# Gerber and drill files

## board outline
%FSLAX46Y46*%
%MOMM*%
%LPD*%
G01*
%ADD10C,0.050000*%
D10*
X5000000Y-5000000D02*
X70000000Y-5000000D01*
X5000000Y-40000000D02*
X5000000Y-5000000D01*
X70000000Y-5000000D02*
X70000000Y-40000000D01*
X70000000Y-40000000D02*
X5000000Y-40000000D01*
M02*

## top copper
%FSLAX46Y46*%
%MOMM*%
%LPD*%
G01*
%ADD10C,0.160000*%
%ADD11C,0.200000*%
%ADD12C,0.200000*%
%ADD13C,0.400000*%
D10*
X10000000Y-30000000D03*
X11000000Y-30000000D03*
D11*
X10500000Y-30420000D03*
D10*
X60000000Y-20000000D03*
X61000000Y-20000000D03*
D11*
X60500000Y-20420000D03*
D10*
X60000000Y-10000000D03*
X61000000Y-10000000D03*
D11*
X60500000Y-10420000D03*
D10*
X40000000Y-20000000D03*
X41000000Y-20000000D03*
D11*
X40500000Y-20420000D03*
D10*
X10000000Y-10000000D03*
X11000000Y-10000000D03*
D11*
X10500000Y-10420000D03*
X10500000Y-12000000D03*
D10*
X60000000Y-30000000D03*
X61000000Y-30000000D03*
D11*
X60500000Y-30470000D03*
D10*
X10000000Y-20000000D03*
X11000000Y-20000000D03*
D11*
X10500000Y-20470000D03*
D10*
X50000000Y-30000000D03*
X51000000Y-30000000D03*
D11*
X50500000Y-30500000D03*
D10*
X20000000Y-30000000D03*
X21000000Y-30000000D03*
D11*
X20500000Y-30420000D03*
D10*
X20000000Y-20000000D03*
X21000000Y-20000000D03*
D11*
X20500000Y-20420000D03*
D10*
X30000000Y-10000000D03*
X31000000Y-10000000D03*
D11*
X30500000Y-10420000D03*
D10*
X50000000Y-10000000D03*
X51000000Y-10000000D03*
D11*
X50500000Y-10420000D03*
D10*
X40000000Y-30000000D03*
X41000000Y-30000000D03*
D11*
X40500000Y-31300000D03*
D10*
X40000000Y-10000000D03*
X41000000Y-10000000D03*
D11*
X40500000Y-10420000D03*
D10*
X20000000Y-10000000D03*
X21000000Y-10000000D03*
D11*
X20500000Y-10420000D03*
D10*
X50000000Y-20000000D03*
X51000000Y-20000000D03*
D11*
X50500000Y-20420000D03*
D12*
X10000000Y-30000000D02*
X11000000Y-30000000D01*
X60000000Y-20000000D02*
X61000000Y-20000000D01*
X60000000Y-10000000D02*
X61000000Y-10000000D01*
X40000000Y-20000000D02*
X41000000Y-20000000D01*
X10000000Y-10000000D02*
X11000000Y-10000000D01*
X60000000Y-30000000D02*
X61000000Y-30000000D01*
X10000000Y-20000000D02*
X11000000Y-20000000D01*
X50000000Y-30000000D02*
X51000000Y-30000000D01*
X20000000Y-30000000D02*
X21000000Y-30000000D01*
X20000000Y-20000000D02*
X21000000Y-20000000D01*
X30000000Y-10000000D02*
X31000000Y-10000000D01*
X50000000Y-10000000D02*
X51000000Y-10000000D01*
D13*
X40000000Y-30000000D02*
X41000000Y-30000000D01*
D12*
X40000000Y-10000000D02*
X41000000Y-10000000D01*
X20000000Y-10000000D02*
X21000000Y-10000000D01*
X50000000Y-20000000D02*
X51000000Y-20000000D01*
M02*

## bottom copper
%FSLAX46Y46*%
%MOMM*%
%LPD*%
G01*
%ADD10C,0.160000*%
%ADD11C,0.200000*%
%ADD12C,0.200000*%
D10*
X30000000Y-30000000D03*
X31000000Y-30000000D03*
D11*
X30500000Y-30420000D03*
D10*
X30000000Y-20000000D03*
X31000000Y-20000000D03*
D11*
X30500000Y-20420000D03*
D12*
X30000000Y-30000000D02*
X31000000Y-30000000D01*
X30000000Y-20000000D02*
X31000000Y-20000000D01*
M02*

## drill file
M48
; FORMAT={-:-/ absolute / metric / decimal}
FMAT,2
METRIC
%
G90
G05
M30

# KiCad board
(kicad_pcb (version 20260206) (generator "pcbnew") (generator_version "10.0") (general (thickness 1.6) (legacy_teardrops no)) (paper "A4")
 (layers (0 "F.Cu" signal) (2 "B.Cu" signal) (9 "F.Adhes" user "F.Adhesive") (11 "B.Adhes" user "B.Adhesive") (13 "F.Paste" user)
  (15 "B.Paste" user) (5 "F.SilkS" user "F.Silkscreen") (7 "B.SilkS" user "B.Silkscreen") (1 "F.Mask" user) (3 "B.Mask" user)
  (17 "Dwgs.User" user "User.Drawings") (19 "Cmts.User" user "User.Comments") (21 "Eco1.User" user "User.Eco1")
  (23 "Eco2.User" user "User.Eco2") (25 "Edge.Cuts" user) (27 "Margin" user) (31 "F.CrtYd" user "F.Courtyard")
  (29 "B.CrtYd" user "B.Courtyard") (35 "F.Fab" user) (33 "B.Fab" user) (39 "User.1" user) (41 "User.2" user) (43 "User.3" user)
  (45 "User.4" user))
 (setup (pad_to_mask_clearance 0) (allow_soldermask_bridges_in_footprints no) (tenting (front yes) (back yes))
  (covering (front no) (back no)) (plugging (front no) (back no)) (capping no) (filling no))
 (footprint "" (layer "F.Cu") (at 10 30)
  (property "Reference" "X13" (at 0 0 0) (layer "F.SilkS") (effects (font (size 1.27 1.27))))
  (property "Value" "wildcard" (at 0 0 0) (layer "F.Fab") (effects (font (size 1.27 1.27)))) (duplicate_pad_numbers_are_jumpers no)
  (pad "1" smd circle (at 0 0) (size 0.16 0.16) (layers "F.Cu") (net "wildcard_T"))
  (pad "2" smd circle (at 1 0) (size 0.16 0.16) (layers "F.Cu") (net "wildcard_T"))
  (pad "3" smd circle (at 0.5 0.42) (size 0.2 0.2) (layers "F.Cu") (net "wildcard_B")))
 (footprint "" (layer "F.Cu") (at 60 20)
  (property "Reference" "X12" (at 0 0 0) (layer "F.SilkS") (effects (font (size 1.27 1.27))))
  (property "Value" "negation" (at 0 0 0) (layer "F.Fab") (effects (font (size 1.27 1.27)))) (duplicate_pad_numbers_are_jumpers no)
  (pad "1" smd circle (at 0 0) (size 0.16 0.16) (layers "F.Cu") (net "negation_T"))
  (pad "2" smd circle (at 1 0) (size 0.16 0.16) (layers "F.Cu") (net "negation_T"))
  (pad "3" smd circle (at 0.5 0.42) (size 0.2 0.2) (layers "F.Cu") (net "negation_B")))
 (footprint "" (layer "F.Cu") (at 60 10)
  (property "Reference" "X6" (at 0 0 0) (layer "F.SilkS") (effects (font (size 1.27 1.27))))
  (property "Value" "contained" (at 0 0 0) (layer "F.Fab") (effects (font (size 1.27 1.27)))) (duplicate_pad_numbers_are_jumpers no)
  (pad "1" smd circle (at 0 0) (size 0.16 0.16) (layers "F.Cu") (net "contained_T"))
  (pad "2" smd circle (at 1 0) (size 0.16 0.16) (layers "F.Cu") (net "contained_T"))
  (pad "3" smd circle (at 0.5 0.42) (size 0.2 0.2) (layers "F.Cu") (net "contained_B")))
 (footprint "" (layer "F.Cu") (at 40 20)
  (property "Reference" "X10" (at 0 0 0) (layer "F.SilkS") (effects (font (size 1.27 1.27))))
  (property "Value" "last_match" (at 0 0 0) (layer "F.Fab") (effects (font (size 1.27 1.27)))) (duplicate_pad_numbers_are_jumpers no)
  (pad "1" smd circle (at 0 0) (size 0.16 0.16) (layers "F.Cu") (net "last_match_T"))
  (pad "2" smd circle (at 1 0) (size 0.16 0.16) (layers "F.Cu") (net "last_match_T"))
  (pad "3" smd circle (at 0.5 0.42) (size 0.2 0.2) (layers "F.Cu") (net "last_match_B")))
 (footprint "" (layer "F.Cu") (at 10 10)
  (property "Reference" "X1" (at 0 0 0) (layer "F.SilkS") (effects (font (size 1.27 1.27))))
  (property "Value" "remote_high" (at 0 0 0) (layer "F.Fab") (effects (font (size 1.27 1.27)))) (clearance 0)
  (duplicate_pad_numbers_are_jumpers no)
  (pad "1" smd circle (at 0 0) (size 0.16 0.16) (layers "F.Cu") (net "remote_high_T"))
  (pad "2" smd circle (at 1 0) (size 0.16 0.16) (layers "F.Cu") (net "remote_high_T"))
  (pad "3" smd circle (at 0.5 0.42) (size 0.2 0.2) (layers "F.Cu") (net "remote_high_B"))
  (pad "4" smd circle (at 0.5 2) (size 0.2 0.2) (layers "F.Cu") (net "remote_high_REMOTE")))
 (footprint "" (layer "F.Cu") (at 60 30)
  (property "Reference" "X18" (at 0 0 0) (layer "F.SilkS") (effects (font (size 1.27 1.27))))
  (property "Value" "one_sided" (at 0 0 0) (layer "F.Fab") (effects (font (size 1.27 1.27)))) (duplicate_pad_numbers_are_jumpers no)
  (pad "1" smd circle (at 0 0) (size 0.16 0.16) (layers "F.Cu") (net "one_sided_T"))
  (pad "2" smd circle (at 1 0) (size 0.16 0.16) (layers "F.Cu") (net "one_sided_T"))
  (pad "3" smd circle (at 0.5 0.47) (size 0.2 0.2) (layers "F.Cu") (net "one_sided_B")))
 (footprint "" (layer "F.Cu") (at 10 20)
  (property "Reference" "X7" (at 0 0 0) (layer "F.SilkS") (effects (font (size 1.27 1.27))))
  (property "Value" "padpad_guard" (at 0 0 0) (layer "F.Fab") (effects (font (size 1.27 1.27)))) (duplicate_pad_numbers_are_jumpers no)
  (pad "1" smd circle (at 0 0) (size 0.16 0.16) (layers "F.Cu") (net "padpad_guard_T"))
  (pad "2" smd circle (at 1 0) (size 0.16 0.16) (layers "F.Cu") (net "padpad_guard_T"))
  (pad "3" smd circle (at 0.5 0.47) (size 0.2 0.2) (layers "F.Cu") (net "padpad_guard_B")))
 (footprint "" (layer "F.Cu") (at 50 30)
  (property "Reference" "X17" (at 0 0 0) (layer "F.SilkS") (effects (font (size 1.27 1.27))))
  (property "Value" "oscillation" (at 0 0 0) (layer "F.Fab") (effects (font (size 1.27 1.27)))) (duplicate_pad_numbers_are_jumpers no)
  (pad "1" smd circle (at 0 0) (size 0.16 0.16) (layers "F.Cu") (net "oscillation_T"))
  (pad "2" smd circle (at 1 0) (size 0.16 0.16) (layers "F.Cu") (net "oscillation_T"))
  (pad "3" smd circle (at 0.5 0.5) (size 0.2 0.2) (layers "F.Cu") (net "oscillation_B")))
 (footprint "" (layer "F.Cu") (at 20 30)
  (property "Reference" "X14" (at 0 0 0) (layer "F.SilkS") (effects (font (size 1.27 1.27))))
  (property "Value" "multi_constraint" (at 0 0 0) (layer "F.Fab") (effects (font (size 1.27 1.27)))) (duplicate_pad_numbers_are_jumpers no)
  (pad "1" smd circle (at 0 0) (size 0.16 0.16) (layers "F.Cu") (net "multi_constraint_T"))
  (pad "2" smd circle (at 1 0) (size 0.16 0.16) (layers "F.Cu") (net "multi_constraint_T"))
  (pad "3" smd circle (at 0.5 0.42) (size 0.2 0.2) (layers "F.Cu") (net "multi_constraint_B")))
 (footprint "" (layer "F.Cu") (at 30 30)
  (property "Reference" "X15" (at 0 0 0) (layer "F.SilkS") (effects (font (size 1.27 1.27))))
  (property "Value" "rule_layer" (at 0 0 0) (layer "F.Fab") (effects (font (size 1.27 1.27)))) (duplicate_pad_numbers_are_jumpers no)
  (pad "1" smd circle (at 0 0) (size 0.16 0.16) (layers "B.Cu") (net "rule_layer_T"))
  (pad "2" smd circle (at 1 0) (size 0.16 0.16) (layers "B.Cu") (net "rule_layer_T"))
  (pad "3" smd circle (at 0.5 0.42) (size 0.2 0.2) (layers "B.Cu") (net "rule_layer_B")))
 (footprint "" (layer "F.Cu") (at 20 20)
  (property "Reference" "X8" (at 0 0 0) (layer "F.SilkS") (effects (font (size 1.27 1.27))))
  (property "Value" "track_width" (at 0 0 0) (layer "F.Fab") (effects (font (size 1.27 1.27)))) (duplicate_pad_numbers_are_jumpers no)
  (pad "1" smd circle (at 0 0) (size 0.16 0.16) (layers "F.Cu") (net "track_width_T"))
  (pad "2" smd circle (at 1 0) (size 0.16 0.16) (layers "F.Cu") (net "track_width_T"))
  (pad "3" smd circle (at 0.5 0.42) (size 0.2 0.2) (layers "F.Cu") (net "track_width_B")))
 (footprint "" (layer "F.Cu") (at 30 10)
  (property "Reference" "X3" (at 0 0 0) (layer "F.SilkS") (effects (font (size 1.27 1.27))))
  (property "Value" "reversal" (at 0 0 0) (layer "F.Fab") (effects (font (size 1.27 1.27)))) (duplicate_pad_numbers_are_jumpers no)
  (pad "1" smd circle (at 0 0) (size 0.16 0.16) (layers "F.Cu") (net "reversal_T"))
  (pad "2" smd circle (at 1 0) (size 0.16 0.16) (layers "F.Cu") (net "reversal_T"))
  (pad "3" smd circle (at 0.5 0.42) (size 0.2 0.2) (layers "F.Cu") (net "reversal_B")))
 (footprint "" (layer "F.Cu") (at 50 10)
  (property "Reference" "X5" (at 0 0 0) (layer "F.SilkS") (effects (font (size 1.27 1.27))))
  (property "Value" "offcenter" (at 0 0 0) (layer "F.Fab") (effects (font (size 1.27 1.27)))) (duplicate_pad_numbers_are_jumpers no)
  (pad "1" smd circle (at 0 0) (size 0.16 0.16) (layers "F.Cu") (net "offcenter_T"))
  (pad "2" smd circle (at 1 0) (size 0.16 0.16) (layers "F.Cu") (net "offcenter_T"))
  (pad "3" smd circle (at 0.5 0.42) (size 0.2 0.2) (layers "F.Cu") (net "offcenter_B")))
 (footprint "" (layer "F.Cu") (at 40 30)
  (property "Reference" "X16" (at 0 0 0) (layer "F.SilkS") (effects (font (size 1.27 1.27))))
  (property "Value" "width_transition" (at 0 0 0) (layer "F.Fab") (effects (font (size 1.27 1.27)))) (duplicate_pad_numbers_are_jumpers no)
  (pad "1" smd circle (at 0 0) (size 0.16 0.16) (layers "F.Cu") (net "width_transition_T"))
  (pad "2" smd circle (at 1 0) (size 0.16 0.16) (layers "F.Cu") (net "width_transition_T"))
  (pad "3" smd circle (at 0.5 1.3) (size 0.2 0.2) (layers "F.Cu") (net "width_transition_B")))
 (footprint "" (layer "F.Cu") (at 30 20)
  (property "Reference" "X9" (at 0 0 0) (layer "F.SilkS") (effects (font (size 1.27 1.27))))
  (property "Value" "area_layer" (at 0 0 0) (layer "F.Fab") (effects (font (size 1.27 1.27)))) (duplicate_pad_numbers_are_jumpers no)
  (pad "1" smd circle (at 0 0) (size 0.16 0.16) (layers "B.Cu") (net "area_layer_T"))
  (pad "2" smd circle (at 1 0) (size 0.16 0.16) (layers "B.Cu") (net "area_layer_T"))
  (pad "3" smd circle (at 0.5 0.42) (size 0.2 0.2) (layers "B.Cu") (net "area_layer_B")))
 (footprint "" (layer "F.Cu") (at 40 10)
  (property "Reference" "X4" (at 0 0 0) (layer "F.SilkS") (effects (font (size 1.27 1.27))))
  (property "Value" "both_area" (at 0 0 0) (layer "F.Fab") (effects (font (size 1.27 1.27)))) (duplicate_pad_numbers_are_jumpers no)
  (pad "1" smd circle (at 0 0) (size 0.16 0.16) (layers "F.Cu") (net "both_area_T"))
  (pad "2" smd circle (at 1 0) (size 0.16 0.16) (layers "F.Cu") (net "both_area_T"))
  (pad "3" smd circle (at 0.5 0.42) (size 0.2 0.2) (layers "F.Cu") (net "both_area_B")))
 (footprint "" (layer "F.Cu") (at 20 10)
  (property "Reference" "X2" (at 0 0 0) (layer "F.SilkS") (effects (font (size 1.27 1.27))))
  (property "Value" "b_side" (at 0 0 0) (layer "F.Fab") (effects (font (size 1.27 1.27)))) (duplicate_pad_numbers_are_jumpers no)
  (pad "1" smd circle (at 0 0) (size 0.16 0.16) (layers "F.Cu") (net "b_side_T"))
  (pad "2" smd circle (at 1 0) (size 0.16 0.16) (layers "F.Cu") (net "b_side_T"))
  (pad "3" smd circle (at 0.5 0.42) (size 0.2 0.2) (layers "F.Cu") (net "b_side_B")))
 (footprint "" (layer "F.Cu") (at 50 20)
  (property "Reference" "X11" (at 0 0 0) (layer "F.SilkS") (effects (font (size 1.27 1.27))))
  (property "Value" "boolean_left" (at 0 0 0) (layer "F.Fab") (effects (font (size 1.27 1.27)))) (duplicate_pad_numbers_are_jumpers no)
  (pad "1" smd circle (at 0 0) (size 0.16 0.16) (layers "F.Cu") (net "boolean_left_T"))
  (pad "2" smd circle (at 1 0) (size 0.16 0.16) (layers "F.Cu") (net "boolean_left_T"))
  (pad "3" smd circle (at 0.5 0.42) (size 0.2 0.2) (layers "F.Cu") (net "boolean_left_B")))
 (gr_line (start 5 5) (end 70 5) (stroke (width 0.05) (type default)) (layer "Edge.Cuts"))
 (gr_line (start 5 40) (end 5 5) (stroke (width 0.05) (type default)) (layer "Edge.Cuts"))
 (gr_line (start 70 5) (end 70 40) (stroke (width 0.05) (type default)) (layer "Edge.Cuts"))
 (gr_line (start 70 40) (end 5 40) (stroke (width 0.05) (type default)) (layer "Edge.Cuts"))
 (segment (start 10 30) (end 11 30) (width 0.2) (layer "F.Cu") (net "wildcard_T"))
 (segment (start 60 20) (end 61 20) (width 0.2) (layer "F.Cu") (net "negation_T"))
 (segment (start 60 10) (end 61 10) (width 0.2) (layer "F.Cu") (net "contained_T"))
 (segment (start 40 20) (end 41 20) (width 0.2) (layer "F.Cu") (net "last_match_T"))
 (segment (start 10 10) (end 11 10) (width 0.2) (layer "F.Cu") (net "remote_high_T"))
 (segment (start 60 30) (end 61 30) (width 0.2) (layer "F.Cu") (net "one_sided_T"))
 (segment (start 10 20) (end 11 20) (width 0.2) (layer "F.Cu") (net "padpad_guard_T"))
 (segment (start 50 30) (end 51 30) (width 0.2) (layer "F.Cu") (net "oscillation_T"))
 (segment (start 20 30) (end 21 30) (width 0.2) (layer "F.Cu") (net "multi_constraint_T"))
 (segment (start 30 30) (end 31 30) (width 0.2) (layer "B.Cu") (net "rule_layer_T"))
 (segment (start 20 20) (end 21 20) (width 0.2) (layer "F.Cu") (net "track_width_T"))
 (segment (start 30 10) (end 31 10) (width 0.2) (layer "F.Cu") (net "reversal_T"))
 (segment (start 50 10) (end 51 10) (width 0.2) (layer "F.Cu") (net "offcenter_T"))
 (segment (start 40 30) (end 41 30) (width 0.4) (layer "F.Cu") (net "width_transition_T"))
 (segment (start 30 20) (end 31 20) (width 0.2) (layer "B.Cu") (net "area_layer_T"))
 (segment (start 40 10) (end 41 10) (width 0.2) (layer "F.Cu") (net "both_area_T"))
 (segment (start 20 10) (end 21 10) (width 0.2) (layer "F.Cu") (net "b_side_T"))
 (segment (start 50 20) (end 51 20) (width 0.2) (layer "F.Cu") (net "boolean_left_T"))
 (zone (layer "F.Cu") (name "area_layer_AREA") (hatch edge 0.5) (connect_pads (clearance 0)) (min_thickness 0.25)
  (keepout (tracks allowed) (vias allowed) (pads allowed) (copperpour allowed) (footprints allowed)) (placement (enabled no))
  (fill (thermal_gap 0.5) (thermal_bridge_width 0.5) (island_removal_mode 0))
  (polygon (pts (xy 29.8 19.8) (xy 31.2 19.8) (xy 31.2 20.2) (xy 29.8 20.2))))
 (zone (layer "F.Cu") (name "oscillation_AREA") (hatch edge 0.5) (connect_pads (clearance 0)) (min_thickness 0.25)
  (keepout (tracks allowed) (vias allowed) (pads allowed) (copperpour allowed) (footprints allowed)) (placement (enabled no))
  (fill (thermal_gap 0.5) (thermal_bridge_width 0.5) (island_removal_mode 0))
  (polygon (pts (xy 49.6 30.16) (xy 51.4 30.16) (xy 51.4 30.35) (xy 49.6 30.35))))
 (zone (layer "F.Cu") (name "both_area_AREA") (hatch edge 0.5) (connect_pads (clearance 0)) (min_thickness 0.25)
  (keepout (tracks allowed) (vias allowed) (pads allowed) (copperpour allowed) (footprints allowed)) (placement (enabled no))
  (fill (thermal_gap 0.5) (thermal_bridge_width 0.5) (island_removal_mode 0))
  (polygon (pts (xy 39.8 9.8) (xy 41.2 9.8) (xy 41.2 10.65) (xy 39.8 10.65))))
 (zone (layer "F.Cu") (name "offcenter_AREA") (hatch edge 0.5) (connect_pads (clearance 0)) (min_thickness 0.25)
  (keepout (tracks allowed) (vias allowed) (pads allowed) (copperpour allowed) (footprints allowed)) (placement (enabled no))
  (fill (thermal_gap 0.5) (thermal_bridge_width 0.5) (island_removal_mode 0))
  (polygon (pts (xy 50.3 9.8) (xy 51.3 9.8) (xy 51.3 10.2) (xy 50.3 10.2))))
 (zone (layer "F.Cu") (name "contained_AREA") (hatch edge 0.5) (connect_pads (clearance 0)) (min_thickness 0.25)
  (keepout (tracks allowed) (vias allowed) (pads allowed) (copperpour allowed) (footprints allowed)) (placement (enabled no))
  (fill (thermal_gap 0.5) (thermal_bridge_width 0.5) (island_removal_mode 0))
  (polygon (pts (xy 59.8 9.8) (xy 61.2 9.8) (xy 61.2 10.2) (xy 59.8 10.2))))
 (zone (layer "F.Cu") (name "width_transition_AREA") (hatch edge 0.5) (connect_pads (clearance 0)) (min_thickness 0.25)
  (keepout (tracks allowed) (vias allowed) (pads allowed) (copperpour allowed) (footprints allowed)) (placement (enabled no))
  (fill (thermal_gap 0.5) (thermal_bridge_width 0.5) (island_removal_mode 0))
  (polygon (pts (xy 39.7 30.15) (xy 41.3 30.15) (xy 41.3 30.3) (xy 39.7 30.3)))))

